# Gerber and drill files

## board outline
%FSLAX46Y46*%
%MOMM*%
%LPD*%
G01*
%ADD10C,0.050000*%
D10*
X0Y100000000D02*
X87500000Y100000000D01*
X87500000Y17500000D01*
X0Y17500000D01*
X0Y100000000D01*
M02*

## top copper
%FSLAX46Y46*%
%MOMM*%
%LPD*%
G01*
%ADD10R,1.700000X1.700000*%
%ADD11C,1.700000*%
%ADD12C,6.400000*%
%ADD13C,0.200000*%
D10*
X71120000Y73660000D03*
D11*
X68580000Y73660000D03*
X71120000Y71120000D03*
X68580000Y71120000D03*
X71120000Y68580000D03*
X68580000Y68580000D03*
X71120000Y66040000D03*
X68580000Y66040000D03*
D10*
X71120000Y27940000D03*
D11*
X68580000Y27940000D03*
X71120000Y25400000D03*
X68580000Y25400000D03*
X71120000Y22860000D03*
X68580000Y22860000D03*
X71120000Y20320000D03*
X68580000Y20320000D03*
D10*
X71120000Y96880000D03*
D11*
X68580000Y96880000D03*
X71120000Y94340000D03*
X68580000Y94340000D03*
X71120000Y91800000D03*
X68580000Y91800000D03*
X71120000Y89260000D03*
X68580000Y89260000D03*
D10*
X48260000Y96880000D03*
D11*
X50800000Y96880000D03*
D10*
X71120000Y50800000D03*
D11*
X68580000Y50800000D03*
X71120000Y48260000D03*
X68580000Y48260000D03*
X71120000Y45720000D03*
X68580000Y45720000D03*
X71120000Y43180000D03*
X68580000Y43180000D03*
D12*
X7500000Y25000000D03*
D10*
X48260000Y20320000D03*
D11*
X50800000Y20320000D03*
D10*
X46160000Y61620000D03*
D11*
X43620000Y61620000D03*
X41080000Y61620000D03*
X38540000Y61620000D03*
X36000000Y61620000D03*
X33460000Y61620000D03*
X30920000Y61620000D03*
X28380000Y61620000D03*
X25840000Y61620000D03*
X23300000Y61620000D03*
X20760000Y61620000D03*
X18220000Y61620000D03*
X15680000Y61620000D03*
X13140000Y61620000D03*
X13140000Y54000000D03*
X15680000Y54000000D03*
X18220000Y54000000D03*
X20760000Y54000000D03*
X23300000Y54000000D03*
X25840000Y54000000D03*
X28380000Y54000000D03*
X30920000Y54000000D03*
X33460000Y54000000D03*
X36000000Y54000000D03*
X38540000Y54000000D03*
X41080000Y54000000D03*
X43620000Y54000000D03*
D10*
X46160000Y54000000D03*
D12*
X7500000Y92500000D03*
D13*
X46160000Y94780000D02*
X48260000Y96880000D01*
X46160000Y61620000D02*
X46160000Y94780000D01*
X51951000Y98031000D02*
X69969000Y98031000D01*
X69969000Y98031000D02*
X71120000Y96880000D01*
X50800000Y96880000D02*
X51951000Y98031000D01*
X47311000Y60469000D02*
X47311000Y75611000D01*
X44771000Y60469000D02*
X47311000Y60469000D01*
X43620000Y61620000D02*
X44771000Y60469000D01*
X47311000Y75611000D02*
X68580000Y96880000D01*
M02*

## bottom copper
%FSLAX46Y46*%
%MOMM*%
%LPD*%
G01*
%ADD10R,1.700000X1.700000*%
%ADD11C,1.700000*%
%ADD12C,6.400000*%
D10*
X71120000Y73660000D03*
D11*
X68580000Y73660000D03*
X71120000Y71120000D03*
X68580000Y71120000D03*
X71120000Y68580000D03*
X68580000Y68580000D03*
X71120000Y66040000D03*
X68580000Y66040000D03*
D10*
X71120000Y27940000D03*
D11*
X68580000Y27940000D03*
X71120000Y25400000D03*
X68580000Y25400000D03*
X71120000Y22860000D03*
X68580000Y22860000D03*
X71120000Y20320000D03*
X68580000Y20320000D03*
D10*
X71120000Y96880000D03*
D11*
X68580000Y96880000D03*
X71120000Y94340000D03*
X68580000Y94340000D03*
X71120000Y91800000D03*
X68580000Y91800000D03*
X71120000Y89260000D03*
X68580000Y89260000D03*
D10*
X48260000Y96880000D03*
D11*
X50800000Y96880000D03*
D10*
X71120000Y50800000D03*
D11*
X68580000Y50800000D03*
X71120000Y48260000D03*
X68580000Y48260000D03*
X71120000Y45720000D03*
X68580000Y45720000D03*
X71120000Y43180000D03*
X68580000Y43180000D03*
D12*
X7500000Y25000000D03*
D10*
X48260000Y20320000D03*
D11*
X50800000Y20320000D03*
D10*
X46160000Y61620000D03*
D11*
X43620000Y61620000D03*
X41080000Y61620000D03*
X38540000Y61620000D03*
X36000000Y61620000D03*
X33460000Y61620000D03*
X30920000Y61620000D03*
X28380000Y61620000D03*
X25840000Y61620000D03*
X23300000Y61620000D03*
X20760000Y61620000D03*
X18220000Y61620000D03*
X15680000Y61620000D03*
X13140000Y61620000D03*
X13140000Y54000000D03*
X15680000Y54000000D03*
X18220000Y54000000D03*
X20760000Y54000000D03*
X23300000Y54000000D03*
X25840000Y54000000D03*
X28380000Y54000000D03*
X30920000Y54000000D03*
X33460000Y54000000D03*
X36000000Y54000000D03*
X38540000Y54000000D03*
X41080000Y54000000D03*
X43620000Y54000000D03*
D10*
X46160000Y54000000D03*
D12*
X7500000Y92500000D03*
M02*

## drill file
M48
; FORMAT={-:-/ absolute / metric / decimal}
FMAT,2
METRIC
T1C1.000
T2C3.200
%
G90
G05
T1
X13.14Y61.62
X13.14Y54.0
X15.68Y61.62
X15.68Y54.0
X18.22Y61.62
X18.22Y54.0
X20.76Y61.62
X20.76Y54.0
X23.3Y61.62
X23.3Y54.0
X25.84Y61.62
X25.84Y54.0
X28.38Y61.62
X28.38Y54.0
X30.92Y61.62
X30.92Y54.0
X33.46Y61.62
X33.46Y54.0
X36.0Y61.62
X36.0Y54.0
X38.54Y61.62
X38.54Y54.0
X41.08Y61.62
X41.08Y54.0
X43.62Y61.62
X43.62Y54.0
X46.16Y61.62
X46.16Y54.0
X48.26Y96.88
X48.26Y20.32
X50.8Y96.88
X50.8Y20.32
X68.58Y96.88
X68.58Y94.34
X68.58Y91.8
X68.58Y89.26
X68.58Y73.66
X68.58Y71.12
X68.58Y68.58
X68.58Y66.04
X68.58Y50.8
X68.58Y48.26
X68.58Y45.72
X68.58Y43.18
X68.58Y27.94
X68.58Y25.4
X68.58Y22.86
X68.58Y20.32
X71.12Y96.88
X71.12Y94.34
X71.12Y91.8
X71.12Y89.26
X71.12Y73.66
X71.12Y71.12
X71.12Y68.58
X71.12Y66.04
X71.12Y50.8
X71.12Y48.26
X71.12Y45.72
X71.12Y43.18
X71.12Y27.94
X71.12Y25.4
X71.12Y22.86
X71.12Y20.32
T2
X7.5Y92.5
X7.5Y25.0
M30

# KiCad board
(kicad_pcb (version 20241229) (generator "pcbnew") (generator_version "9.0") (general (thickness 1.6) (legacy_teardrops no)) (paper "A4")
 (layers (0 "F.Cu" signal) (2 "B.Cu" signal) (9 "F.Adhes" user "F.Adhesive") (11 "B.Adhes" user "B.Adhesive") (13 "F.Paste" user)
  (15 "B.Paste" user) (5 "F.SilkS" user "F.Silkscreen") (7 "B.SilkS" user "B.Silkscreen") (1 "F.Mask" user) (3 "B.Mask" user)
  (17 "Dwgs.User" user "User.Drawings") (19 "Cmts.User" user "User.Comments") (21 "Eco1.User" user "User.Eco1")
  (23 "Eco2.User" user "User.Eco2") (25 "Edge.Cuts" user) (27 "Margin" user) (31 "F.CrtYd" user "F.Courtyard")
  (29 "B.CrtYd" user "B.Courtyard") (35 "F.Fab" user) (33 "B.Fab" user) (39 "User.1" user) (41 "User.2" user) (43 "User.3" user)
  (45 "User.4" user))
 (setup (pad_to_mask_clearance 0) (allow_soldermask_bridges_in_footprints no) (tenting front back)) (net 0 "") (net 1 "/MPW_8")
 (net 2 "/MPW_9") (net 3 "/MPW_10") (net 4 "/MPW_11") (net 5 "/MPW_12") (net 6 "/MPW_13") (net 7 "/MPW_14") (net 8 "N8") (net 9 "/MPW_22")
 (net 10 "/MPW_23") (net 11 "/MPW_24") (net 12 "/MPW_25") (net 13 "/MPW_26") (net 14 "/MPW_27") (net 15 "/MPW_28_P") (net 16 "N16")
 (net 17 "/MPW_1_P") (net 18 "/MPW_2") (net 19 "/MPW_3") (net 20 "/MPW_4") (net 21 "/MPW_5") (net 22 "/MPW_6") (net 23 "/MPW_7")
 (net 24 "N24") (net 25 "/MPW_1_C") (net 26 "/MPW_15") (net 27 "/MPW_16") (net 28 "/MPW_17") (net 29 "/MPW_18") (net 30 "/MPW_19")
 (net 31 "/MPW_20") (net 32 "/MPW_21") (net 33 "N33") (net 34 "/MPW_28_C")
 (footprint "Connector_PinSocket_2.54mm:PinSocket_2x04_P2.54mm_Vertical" (layer "F.Cu") (at 71.12 -73.66)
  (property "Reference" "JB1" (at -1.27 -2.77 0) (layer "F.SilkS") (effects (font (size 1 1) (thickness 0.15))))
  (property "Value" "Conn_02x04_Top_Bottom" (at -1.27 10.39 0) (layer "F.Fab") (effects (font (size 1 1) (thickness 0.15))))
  (pad "1" thru_hole rect (at 0 0) (size 1.7 1.7) (drill 1) (layers "*.Cu" "*.Mask") (remove_unused_layers no) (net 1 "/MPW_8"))
  (pad "2" thru_hole circle (at -2.54 0) (size 1.7 1.7) (drill 1) (layers "*.Cu" "*.Mask") (remove_unused_layers no) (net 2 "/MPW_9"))
  (pad "3" thru_hole circle (at 0 2.54) (size 1.7 1.7) (drill 1) (layers "*.Cu" "*.Mask") (remove_unused_layers no) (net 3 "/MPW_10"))
  (pad "4" thru_hole circle (at -2.54 2.54) (size 1.7 1.7) (drill 1) (layers "*.Cu" "*.Mask") (remove_unused_layers no) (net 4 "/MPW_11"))
  (pad "5" thru_hole circle (at 0 5.08) (size 1.7 1.7) (drill 1) (layers "*.Cu" "*.Mask") (remove_unused_layers no) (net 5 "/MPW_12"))
  (pad "6" thru_hole circle (at -2.54 5.08) (size 1.7 1.7) (drill 1) (layers "*.Cu" "*.Mask") (remove_unused_layers no) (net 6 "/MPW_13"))
  (pad "7" thru_hole circle (at 0 7.62) (size 1.7 1.7) (drill 1) (layers "*.Cu" "*.Mask") (remove_unused_layers no) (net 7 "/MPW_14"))
  (pad "8" thru_hole circle (at -2.54 7.62) (size 1.7 1.7) (drill 1) (layers "*.Cu" "*.Mask") (remove_unused_layers no) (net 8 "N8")))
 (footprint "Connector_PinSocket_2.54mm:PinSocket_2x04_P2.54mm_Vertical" (layer "F.Cu") (at 71.12 -27.94)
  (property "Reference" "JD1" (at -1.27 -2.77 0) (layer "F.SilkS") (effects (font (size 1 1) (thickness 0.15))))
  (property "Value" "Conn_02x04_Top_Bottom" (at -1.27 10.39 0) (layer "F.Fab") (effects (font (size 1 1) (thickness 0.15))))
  (pad "1" thru_hole rect (at 0 0) (size 1.7 1.7) (drill 1) (layers "*.Cu" "*.Mask") (remove_unused_layers no) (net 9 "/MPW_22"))
  (pad "2" thru_hole circle (at -2.54 0) (size 1.7 1.7) (drill 1) (layers "*.Cu" "*.Mask") (remove_unused_layers no) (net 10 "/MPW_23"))
  (pad "3" thru_hole circle (at 0 2.54) (size 1.7 1.7) (drill 1) (layers "*.Cu" "*.Mask") (remove_unused_layers no) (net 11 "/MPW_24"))
  (pad "4" thru_hole circle (at -2.54 2.54) (size 1.7 1.7) (drill 1) (layers "*.Cu" "*.Mask") (remove_unused_layers no) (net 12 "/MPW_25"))
  (pad "5" thru_hole circle (at 0 5.08) (size 1.7 1.7) (drill 1) (layers "*.Cu" "*.Mask") (remove_unused_layers no) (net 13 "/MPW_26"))
  (pad "6" thru_hole circle (at -2.54 5.08) (size 1.7 1.7) (drill 1) (layers "*.Cu" "*.Mask") (remove_unused_layers no) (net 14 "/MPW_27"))
  (pad "7" thru_hole circle (at 0 7.62) (size 1.7 1.7) (drill 1) (layers "*.Cu" "*.Mask") (remove_unused_layers no) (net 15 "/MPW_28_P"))
  (pad "8" thru_hole circle (at -2.54 7.62) (size 1.7 1.7) (drill 1) (layers "*.Cu" "*.Mask") (remove_unused_layers no) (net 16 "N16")))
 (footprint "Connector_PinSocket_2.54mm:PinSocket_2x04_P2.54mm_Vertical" (layer "F.Cu") (at 71.12 -96.88)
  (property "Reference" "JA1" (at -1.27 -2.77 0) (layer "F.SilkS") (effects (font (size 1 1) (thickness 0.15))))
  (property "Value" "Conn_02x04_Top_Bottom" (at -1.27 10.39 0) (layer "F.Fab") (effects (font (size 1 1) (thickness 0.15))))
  (pad "1" thru_hole rect (at 0 0) (size 1.7 1.7) (drill 1) (layers "*.Cu" "*.Mask") (remove_unused_layers no) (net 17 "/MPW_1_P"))
  (pad "2" thru_hole circle (at -2.54 0) (size 1.7 1.7) (drill 1) (layers "*.Cu" "*.Mask") (remove_unused_layers no) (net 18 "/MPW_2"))
  (pad "3" thru_hole circle (at 0 2.54) (size 1.7 1.7) (drill 1) (layers "*.Cu" "*.Mask") (remove_unused_layers no) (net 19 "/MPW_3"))
  (pad "4" thru_hole circle (at -2.54 2.54) (size 1.7 1.7) (drill 1) (layers "*.Cu" "*.Mask") (remove_unused_layers no) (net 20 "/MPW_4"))
  (pad "5" thru_hole circle (at 0 5.08) (size 1.7 1.7) (drill 1) (layers "*.Cu" "*.Mask") (remove_unused_layers no) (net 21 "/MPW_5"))
  (pad "6" thru_hole circle (at -2.54 5.08) (size 1.7 1.7) (drill 1) (layers "*.Cu" "*.Mask") (remove_unused_layers no) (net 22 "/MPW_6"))
  (pad "7" thru_hole circle (at 0 7.62) (size 1.7 1.7) (drill 1) (layers "*.Cu" "*.Mask") (remove_unused_layers no) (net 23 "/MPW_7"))
  (pad "8" thru_hole circle (at -2.54 7.62) (size 1.7 1.7) (drill 1) (layers "*.Cu" "*.Mask") (remove_unused_layers no) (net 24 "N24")))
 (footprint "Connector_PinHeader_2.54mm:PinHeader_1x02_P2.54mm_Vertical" (layer "F.Cu") (at 48.26 -96.88 90)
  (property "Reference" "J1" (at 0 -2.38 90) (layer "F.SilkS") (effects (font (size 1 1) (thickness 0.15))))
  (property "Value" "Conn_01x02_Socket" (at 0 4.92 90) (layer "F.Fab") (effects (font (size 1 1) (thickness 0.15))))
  (pad "1" thru_hole rect (at 0 0 90) (size 1.7 1.7) (drill 1) (layers "*.Cu" "*.Mask") (remove_unused_layers no) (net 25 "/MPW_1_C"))
  (pad "2" thru_hole circle (at 0 2.54 90) (size 1.7 1.7) (drill 1) (layers "*.Cu" "*.Mask") (remove_unused_layers no) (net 17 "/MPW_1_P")))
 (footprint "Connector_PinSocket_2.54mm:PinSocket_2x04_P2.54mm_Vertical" (layer "F.Cu") (at 71.12 -50.8)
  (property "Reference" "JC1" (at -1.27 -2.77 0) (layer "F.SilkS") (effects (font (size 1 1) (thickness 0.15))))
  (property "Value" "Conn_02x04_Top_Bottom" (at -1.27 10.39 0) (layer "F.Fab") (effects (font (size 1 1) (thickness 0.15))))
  (pad "1" thru_hole rect (at 0 0) (size 1.7 1.7) (drill 1) (layers "*.Cu" "*.Mask") (remove_unused_layers no) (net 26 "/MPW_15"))
  (pad "2" thru_hole circle (at -2.54 0) (size 1.7 1.7) (drill 1) (layers "*.Cu" "*.Mask") (remove_unused_layers no) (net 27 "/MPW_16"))
  (pad "3" thru_hole circle (at 0 2.54) (size 1.7 1.7) (drill 1) (layers "*.Cu" "*.Mask") (remove_unused_layers no) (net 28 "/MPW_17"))
  (pad "4" thru_hole circle (at -2.54 2.54) (size 1.7 1.7) (drill 1) (layers "*.Cu" "*.Mask") (remove_unused_layers no) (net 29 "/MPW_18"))
  (pad "5" thru_hole circle (at 0 5.08) (size 1.7 1.7) (drill 1) (layers "*.Cu" "*.Mask") (remove_unused_layers no) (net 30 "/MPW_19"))
  (pad "6" thru_hole circle (at -2.54 5.08) (size 1.7 1.7) (drill 1) (layers "*.Cu" "*.Mask") (remove_unused_layers no) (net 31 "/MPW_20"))
  (pad "7" thru_hole circle (at 0 7.62) (size 1.7 1.7) (drill 1) (layers "*.Cu" "*.Mask") (remove_unused_layers no) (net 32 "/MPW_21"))
  (pad "8" thru_hole circle (at -2.54 7.62) (size 1.7 1.7) (drill 1) (layers "*.Cu" "*.Mask") (remove_unused_layers no) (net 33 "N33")))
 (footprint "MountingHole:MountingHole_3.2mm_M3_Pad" (layer "F.Cu") (at 7.5 -25)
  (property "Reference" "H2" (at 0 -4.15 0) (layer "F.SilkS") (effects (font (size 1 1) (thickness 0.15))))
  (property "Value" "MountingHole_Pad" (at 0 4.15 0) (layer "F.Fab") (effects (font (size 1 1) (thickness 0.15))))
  (pad "1" thru_hole circle (at 0 0) (size 6.4 6.4) (drill 3.2) (layers "*.Cu" "*.Mask") (remove_unused_layers no) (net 15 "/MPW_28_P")
   (zone_connect 2)))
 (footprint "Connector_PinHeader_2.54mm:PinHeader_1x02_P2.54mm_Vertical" (layer "F.Cu") (at 48.26 -20.32 90)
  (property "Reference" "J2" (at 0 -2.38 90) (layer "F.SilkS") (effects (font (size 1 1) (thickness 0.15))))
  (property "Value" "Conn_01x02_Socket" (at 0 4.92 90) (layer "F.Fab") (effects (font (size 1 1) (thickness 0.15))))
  (pad "1" thru_hole rect (at 0 0 90) (size 1.7 1.7) (drill 1) (layers "*.Cu" "*.Mask") (remove_unused_layers no) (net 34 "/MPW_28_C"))
  (pad "2" thru_hole circle (at 0 2.54 90) (size 1.7 1.7) (drill 1) (layers "*.Cu" "*.Mask") (remove_unused_layers no) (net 15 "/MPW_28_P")))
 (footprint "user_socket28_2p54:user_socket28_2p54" (layer "F.Cu") (at 47.96 -59.87 -90)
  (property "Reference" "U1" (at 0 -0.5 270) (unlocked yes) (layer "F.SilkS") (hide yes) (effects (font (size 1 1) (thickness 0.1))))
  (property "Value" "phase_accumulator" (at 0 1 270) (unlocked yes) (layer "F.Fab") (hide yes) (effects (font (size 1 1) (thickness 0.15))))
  (pad "1" thru_hole rect (at -1.75 1.8 270) (size 1.7 1.7) (drill 1) (layers "*.Cu" "*.Mask") (remove_unused_layers no) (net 25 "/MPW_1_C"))
  (pad "2" thru_hole circle (at -1.75 4.34 270) (size 1.7 1.7) (drill 1) (layers "*.Cu" "*.Mask") (remove_unused_layers no)
   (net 18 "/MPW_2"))
  (pad "3" thru_hole circle (at -1.75 6.88 270) (size 1.7 1.7) (drill 1) (layers "*.Cu" "*.Mask") (remove_unused_layers no)
   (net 19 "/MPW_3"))
  (pad "4" thru_hole circle (at -1.75 9.42 270) (size 1.7 1.7) (drill 1) (layers "*.Cu" "*.Mask") (remove_unused_layers no)
   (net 20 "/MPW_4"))
  (pad "5" thru_hole circle (at -1.75 11.96 270) (size 1.7 1.7) (drill 1) (layers "*.Cu" "*.Mask") (remove_unused_layers no)
   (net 21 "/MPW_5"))
  (pad "6" thru_hole circle (at -1.75 14.5 270) (size 1.7 1.7) (drill 1) (layers "*.Cu" "*.Mask") (remove_unused_layers no)
   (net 22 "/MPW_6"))
  (pad "7" thru_hole circle (at -1.75 17.04 270) (size 1.7 1.7) (drill 1) (layers "*.Cu" "*.Mask") (remove_unused_layers no)
   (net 23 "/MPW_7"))
  (pad "8" thru_hole circle (at -1.75 19.58 270) (size 1.7 1.7) (drill 1) (layers "*.Cu" "*.Mask") (remove_unused_layers no)
   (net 1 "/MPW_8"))
  (pad "9" thru_hole circle (at -1.75 22.12 270) (size 1.7 1.7) (drill 1) (layers "*.Cu" "*.Mask") (remove_unused_layers no)
   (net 2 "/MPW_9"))
  (pad "10" thru_hole circle (at -1.75 24.66 270) (size 1.7 1.7) (drill 1) (layers "*.Cu" "*.Mask") (remove_unused_layers no)
   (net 3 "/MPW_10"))
  (pad "11" thru_hole circle (at -1.75 27.2 270) (size 1.7 1.7) (drill 1) (layers "*.Cu" "*.Mask") (remove_unused_layers no)
   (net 4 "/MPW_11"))
  (pad "12" thru_hole circle (at -1.75 29.74 270) (size 1.7 1.7) (drill 1) (layers "*.Cu" "*.Mask") (remove_unused_layers no)
   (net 5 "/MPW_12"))
  (pad "13" thru_hole circle (at -1.75 32.28 270) (size 1.7 1.7) (drill 1) (layers "*.Cu" "*.Mask") (remove_unused_layers no)
   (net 6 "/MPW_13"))
  (pad "14" thru_hole circle (at -1.75 34.82 270) (size 1.7 1.7) (drill 1) (layers "*.Cu" "*.Mask") (remove_unused_layers no)
   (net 7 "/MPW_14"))
  (pad "15" thru_hole circle (at 5.87 34.82 270) (size 1.7 1.7) (drill 1) (layers "*.Cu" "*.Mask") (remove_unused_layers no)
   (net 26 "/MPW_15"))
  (pad "16" thru_hole circle (at 5.87 32.28 270) (size 1.7 1.7) (drill 1) (layers "*.Cu" "*.Mask") (remove_unused_layers no)
   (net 27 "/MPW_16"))
  (pad "17" thru_hole circle (at 5.87 29.74 270) (size 1.7 1.7) (drill 1) (layers "*.Cu" "*.Mask") (remove_unused_layers no)
   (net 28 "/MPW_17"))
  (pad "18" thru_hole circle (at 5.87 27.2 270) (size 1.7 1.7) (drill 1) (layers "*.Cu" "*.Mask") (remove_unused_layers no)
   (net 29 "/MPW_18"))
  (pad "19" thru_hole circle (at 5.87 24.66 270) (size 1.7 1.7) (drill 1) (layers "*.Cu" "*.Mask") (remove_unused_layers no)
   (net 30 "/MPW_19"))
  (pad "20" thru_hole circle (at 5.87 22.12 270) (size 1.7 1.7) (drill 1) (layers "*.Cu" "*.Mask") (remove_unused_layers no)
   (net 31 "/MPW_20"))
  (pad "21" thru_hole circle (at 5.87 19.58 270) (size 1.7 1.7) (drill 1) (layers "*.Cu" "*.Mask") (remove_unused_layers no)
   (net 32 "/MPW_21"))
  (pad "22" thru_hole circle (at 5.87 17.04 270) (size 1.7 1.7) (drill 1) (layers "*.Cu" "*.Mask") (remove_unused_layers no)
   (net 9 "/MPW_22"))
  (pad "23" thru_hole circle (at 5.87 14.5 270) (size 1.7 1.7) (drill 1) (layers "*.Cu" "*.Mask") (remove_unused_layers no)
   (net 10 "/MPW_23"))
  (pad "24" thru_hole circle (at 5.87 11.96 270) (size 1.7 1.7) (drill 1) (layers "*.Cu" "*.Mask") (remove_unused_layers no)
   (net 11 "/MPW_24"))
  (pad "25" thru_hole circle (at 5.87 9.42 270) (size 1.7 1.7) (drill 1) (layers "*.Cu" "*.Mask") (remove_unused_layers no)
   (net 12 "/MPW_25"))
  (pad "26" thru_hole circle (at 5.87 6.88 270) (size 1.7 1.7) (drill 1) (layers "*.Cu" "*.Mask") (remove_unused_layers no)
   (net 13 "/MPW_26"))
  (pad "27" thru_hole circle (at 5.87 4.34 270) (size 1.7 1.7) (drill 1) (layers "*.Cu" "*.Mask") (remove_unused_layers no)
   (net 14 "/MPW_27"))
  (pad "28" thru_hole rect (at 5.87 1.8 270) (size 1.7 1.7) (drill 1) (layers "*.Cu" "*.Mask") (remove_unused_layers no)
   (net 34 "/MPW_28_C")))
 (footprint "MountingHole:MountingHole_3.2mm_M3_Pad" (layer "F.Cu") (at 7.5 -92.5)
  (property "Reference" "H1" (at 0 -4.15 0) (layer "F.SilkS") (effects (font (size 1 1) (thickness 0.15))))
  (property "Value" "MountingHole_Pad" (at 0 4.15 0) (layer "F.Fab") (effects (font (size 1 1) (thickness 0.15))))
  (pad "1" thru_hole circle (at 0 0) (size 6.4 6.4) (drill 3.2) (layers "*.Cu" "*.Mask") (remove_unused_layers no) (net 15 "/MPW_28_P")
   (zone_connect 2)))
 (gr_rect (start 0 -100) (end 87.5 -17.5) (stroke (width 0.05) (type default)) (fill no) (layer "Edge.Cuts"))
 (segment (start 46.16 -94.78) (end 48.26 -96.88) (width 0.2) (layer "F.Cu") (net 25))
 (segment (start 46.16 -61.62) (end 46.16 -94.78) (width 0.2) (layer "F.Cu") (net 25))
 (segment (start 51.951 -98.031) (end 69.969 -98.031) (width 0.2) (layer "F.Cu") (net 17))
 (segment (start 69.969 -98.031) (end 71.12 -96.88) (width 0.2) (layer "F.Cu") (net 17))
 (segment (start 50.8 -96.88) (end 51.951 -98.031) (width 0.2) (layer "F.Cu") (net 17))
 (segment (start 47.311 -60.469) (end 47.311 -75.611) (width 0.2) (layer "F.Cu") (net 18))
 (segment (start 44.771 -60.469) (end 47.311 -60.469) (width 0.2) (layer "F.Cu") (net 18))
 (segment (start 43.62 -61.62) (end 44.771 -60.469) (width 0.2) (layer "F.Cu") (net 18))
 (segment (start 47.311 -75.611) (end 68.58 -96.88) (width 0.2) (layer "F.Cu") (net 18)))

